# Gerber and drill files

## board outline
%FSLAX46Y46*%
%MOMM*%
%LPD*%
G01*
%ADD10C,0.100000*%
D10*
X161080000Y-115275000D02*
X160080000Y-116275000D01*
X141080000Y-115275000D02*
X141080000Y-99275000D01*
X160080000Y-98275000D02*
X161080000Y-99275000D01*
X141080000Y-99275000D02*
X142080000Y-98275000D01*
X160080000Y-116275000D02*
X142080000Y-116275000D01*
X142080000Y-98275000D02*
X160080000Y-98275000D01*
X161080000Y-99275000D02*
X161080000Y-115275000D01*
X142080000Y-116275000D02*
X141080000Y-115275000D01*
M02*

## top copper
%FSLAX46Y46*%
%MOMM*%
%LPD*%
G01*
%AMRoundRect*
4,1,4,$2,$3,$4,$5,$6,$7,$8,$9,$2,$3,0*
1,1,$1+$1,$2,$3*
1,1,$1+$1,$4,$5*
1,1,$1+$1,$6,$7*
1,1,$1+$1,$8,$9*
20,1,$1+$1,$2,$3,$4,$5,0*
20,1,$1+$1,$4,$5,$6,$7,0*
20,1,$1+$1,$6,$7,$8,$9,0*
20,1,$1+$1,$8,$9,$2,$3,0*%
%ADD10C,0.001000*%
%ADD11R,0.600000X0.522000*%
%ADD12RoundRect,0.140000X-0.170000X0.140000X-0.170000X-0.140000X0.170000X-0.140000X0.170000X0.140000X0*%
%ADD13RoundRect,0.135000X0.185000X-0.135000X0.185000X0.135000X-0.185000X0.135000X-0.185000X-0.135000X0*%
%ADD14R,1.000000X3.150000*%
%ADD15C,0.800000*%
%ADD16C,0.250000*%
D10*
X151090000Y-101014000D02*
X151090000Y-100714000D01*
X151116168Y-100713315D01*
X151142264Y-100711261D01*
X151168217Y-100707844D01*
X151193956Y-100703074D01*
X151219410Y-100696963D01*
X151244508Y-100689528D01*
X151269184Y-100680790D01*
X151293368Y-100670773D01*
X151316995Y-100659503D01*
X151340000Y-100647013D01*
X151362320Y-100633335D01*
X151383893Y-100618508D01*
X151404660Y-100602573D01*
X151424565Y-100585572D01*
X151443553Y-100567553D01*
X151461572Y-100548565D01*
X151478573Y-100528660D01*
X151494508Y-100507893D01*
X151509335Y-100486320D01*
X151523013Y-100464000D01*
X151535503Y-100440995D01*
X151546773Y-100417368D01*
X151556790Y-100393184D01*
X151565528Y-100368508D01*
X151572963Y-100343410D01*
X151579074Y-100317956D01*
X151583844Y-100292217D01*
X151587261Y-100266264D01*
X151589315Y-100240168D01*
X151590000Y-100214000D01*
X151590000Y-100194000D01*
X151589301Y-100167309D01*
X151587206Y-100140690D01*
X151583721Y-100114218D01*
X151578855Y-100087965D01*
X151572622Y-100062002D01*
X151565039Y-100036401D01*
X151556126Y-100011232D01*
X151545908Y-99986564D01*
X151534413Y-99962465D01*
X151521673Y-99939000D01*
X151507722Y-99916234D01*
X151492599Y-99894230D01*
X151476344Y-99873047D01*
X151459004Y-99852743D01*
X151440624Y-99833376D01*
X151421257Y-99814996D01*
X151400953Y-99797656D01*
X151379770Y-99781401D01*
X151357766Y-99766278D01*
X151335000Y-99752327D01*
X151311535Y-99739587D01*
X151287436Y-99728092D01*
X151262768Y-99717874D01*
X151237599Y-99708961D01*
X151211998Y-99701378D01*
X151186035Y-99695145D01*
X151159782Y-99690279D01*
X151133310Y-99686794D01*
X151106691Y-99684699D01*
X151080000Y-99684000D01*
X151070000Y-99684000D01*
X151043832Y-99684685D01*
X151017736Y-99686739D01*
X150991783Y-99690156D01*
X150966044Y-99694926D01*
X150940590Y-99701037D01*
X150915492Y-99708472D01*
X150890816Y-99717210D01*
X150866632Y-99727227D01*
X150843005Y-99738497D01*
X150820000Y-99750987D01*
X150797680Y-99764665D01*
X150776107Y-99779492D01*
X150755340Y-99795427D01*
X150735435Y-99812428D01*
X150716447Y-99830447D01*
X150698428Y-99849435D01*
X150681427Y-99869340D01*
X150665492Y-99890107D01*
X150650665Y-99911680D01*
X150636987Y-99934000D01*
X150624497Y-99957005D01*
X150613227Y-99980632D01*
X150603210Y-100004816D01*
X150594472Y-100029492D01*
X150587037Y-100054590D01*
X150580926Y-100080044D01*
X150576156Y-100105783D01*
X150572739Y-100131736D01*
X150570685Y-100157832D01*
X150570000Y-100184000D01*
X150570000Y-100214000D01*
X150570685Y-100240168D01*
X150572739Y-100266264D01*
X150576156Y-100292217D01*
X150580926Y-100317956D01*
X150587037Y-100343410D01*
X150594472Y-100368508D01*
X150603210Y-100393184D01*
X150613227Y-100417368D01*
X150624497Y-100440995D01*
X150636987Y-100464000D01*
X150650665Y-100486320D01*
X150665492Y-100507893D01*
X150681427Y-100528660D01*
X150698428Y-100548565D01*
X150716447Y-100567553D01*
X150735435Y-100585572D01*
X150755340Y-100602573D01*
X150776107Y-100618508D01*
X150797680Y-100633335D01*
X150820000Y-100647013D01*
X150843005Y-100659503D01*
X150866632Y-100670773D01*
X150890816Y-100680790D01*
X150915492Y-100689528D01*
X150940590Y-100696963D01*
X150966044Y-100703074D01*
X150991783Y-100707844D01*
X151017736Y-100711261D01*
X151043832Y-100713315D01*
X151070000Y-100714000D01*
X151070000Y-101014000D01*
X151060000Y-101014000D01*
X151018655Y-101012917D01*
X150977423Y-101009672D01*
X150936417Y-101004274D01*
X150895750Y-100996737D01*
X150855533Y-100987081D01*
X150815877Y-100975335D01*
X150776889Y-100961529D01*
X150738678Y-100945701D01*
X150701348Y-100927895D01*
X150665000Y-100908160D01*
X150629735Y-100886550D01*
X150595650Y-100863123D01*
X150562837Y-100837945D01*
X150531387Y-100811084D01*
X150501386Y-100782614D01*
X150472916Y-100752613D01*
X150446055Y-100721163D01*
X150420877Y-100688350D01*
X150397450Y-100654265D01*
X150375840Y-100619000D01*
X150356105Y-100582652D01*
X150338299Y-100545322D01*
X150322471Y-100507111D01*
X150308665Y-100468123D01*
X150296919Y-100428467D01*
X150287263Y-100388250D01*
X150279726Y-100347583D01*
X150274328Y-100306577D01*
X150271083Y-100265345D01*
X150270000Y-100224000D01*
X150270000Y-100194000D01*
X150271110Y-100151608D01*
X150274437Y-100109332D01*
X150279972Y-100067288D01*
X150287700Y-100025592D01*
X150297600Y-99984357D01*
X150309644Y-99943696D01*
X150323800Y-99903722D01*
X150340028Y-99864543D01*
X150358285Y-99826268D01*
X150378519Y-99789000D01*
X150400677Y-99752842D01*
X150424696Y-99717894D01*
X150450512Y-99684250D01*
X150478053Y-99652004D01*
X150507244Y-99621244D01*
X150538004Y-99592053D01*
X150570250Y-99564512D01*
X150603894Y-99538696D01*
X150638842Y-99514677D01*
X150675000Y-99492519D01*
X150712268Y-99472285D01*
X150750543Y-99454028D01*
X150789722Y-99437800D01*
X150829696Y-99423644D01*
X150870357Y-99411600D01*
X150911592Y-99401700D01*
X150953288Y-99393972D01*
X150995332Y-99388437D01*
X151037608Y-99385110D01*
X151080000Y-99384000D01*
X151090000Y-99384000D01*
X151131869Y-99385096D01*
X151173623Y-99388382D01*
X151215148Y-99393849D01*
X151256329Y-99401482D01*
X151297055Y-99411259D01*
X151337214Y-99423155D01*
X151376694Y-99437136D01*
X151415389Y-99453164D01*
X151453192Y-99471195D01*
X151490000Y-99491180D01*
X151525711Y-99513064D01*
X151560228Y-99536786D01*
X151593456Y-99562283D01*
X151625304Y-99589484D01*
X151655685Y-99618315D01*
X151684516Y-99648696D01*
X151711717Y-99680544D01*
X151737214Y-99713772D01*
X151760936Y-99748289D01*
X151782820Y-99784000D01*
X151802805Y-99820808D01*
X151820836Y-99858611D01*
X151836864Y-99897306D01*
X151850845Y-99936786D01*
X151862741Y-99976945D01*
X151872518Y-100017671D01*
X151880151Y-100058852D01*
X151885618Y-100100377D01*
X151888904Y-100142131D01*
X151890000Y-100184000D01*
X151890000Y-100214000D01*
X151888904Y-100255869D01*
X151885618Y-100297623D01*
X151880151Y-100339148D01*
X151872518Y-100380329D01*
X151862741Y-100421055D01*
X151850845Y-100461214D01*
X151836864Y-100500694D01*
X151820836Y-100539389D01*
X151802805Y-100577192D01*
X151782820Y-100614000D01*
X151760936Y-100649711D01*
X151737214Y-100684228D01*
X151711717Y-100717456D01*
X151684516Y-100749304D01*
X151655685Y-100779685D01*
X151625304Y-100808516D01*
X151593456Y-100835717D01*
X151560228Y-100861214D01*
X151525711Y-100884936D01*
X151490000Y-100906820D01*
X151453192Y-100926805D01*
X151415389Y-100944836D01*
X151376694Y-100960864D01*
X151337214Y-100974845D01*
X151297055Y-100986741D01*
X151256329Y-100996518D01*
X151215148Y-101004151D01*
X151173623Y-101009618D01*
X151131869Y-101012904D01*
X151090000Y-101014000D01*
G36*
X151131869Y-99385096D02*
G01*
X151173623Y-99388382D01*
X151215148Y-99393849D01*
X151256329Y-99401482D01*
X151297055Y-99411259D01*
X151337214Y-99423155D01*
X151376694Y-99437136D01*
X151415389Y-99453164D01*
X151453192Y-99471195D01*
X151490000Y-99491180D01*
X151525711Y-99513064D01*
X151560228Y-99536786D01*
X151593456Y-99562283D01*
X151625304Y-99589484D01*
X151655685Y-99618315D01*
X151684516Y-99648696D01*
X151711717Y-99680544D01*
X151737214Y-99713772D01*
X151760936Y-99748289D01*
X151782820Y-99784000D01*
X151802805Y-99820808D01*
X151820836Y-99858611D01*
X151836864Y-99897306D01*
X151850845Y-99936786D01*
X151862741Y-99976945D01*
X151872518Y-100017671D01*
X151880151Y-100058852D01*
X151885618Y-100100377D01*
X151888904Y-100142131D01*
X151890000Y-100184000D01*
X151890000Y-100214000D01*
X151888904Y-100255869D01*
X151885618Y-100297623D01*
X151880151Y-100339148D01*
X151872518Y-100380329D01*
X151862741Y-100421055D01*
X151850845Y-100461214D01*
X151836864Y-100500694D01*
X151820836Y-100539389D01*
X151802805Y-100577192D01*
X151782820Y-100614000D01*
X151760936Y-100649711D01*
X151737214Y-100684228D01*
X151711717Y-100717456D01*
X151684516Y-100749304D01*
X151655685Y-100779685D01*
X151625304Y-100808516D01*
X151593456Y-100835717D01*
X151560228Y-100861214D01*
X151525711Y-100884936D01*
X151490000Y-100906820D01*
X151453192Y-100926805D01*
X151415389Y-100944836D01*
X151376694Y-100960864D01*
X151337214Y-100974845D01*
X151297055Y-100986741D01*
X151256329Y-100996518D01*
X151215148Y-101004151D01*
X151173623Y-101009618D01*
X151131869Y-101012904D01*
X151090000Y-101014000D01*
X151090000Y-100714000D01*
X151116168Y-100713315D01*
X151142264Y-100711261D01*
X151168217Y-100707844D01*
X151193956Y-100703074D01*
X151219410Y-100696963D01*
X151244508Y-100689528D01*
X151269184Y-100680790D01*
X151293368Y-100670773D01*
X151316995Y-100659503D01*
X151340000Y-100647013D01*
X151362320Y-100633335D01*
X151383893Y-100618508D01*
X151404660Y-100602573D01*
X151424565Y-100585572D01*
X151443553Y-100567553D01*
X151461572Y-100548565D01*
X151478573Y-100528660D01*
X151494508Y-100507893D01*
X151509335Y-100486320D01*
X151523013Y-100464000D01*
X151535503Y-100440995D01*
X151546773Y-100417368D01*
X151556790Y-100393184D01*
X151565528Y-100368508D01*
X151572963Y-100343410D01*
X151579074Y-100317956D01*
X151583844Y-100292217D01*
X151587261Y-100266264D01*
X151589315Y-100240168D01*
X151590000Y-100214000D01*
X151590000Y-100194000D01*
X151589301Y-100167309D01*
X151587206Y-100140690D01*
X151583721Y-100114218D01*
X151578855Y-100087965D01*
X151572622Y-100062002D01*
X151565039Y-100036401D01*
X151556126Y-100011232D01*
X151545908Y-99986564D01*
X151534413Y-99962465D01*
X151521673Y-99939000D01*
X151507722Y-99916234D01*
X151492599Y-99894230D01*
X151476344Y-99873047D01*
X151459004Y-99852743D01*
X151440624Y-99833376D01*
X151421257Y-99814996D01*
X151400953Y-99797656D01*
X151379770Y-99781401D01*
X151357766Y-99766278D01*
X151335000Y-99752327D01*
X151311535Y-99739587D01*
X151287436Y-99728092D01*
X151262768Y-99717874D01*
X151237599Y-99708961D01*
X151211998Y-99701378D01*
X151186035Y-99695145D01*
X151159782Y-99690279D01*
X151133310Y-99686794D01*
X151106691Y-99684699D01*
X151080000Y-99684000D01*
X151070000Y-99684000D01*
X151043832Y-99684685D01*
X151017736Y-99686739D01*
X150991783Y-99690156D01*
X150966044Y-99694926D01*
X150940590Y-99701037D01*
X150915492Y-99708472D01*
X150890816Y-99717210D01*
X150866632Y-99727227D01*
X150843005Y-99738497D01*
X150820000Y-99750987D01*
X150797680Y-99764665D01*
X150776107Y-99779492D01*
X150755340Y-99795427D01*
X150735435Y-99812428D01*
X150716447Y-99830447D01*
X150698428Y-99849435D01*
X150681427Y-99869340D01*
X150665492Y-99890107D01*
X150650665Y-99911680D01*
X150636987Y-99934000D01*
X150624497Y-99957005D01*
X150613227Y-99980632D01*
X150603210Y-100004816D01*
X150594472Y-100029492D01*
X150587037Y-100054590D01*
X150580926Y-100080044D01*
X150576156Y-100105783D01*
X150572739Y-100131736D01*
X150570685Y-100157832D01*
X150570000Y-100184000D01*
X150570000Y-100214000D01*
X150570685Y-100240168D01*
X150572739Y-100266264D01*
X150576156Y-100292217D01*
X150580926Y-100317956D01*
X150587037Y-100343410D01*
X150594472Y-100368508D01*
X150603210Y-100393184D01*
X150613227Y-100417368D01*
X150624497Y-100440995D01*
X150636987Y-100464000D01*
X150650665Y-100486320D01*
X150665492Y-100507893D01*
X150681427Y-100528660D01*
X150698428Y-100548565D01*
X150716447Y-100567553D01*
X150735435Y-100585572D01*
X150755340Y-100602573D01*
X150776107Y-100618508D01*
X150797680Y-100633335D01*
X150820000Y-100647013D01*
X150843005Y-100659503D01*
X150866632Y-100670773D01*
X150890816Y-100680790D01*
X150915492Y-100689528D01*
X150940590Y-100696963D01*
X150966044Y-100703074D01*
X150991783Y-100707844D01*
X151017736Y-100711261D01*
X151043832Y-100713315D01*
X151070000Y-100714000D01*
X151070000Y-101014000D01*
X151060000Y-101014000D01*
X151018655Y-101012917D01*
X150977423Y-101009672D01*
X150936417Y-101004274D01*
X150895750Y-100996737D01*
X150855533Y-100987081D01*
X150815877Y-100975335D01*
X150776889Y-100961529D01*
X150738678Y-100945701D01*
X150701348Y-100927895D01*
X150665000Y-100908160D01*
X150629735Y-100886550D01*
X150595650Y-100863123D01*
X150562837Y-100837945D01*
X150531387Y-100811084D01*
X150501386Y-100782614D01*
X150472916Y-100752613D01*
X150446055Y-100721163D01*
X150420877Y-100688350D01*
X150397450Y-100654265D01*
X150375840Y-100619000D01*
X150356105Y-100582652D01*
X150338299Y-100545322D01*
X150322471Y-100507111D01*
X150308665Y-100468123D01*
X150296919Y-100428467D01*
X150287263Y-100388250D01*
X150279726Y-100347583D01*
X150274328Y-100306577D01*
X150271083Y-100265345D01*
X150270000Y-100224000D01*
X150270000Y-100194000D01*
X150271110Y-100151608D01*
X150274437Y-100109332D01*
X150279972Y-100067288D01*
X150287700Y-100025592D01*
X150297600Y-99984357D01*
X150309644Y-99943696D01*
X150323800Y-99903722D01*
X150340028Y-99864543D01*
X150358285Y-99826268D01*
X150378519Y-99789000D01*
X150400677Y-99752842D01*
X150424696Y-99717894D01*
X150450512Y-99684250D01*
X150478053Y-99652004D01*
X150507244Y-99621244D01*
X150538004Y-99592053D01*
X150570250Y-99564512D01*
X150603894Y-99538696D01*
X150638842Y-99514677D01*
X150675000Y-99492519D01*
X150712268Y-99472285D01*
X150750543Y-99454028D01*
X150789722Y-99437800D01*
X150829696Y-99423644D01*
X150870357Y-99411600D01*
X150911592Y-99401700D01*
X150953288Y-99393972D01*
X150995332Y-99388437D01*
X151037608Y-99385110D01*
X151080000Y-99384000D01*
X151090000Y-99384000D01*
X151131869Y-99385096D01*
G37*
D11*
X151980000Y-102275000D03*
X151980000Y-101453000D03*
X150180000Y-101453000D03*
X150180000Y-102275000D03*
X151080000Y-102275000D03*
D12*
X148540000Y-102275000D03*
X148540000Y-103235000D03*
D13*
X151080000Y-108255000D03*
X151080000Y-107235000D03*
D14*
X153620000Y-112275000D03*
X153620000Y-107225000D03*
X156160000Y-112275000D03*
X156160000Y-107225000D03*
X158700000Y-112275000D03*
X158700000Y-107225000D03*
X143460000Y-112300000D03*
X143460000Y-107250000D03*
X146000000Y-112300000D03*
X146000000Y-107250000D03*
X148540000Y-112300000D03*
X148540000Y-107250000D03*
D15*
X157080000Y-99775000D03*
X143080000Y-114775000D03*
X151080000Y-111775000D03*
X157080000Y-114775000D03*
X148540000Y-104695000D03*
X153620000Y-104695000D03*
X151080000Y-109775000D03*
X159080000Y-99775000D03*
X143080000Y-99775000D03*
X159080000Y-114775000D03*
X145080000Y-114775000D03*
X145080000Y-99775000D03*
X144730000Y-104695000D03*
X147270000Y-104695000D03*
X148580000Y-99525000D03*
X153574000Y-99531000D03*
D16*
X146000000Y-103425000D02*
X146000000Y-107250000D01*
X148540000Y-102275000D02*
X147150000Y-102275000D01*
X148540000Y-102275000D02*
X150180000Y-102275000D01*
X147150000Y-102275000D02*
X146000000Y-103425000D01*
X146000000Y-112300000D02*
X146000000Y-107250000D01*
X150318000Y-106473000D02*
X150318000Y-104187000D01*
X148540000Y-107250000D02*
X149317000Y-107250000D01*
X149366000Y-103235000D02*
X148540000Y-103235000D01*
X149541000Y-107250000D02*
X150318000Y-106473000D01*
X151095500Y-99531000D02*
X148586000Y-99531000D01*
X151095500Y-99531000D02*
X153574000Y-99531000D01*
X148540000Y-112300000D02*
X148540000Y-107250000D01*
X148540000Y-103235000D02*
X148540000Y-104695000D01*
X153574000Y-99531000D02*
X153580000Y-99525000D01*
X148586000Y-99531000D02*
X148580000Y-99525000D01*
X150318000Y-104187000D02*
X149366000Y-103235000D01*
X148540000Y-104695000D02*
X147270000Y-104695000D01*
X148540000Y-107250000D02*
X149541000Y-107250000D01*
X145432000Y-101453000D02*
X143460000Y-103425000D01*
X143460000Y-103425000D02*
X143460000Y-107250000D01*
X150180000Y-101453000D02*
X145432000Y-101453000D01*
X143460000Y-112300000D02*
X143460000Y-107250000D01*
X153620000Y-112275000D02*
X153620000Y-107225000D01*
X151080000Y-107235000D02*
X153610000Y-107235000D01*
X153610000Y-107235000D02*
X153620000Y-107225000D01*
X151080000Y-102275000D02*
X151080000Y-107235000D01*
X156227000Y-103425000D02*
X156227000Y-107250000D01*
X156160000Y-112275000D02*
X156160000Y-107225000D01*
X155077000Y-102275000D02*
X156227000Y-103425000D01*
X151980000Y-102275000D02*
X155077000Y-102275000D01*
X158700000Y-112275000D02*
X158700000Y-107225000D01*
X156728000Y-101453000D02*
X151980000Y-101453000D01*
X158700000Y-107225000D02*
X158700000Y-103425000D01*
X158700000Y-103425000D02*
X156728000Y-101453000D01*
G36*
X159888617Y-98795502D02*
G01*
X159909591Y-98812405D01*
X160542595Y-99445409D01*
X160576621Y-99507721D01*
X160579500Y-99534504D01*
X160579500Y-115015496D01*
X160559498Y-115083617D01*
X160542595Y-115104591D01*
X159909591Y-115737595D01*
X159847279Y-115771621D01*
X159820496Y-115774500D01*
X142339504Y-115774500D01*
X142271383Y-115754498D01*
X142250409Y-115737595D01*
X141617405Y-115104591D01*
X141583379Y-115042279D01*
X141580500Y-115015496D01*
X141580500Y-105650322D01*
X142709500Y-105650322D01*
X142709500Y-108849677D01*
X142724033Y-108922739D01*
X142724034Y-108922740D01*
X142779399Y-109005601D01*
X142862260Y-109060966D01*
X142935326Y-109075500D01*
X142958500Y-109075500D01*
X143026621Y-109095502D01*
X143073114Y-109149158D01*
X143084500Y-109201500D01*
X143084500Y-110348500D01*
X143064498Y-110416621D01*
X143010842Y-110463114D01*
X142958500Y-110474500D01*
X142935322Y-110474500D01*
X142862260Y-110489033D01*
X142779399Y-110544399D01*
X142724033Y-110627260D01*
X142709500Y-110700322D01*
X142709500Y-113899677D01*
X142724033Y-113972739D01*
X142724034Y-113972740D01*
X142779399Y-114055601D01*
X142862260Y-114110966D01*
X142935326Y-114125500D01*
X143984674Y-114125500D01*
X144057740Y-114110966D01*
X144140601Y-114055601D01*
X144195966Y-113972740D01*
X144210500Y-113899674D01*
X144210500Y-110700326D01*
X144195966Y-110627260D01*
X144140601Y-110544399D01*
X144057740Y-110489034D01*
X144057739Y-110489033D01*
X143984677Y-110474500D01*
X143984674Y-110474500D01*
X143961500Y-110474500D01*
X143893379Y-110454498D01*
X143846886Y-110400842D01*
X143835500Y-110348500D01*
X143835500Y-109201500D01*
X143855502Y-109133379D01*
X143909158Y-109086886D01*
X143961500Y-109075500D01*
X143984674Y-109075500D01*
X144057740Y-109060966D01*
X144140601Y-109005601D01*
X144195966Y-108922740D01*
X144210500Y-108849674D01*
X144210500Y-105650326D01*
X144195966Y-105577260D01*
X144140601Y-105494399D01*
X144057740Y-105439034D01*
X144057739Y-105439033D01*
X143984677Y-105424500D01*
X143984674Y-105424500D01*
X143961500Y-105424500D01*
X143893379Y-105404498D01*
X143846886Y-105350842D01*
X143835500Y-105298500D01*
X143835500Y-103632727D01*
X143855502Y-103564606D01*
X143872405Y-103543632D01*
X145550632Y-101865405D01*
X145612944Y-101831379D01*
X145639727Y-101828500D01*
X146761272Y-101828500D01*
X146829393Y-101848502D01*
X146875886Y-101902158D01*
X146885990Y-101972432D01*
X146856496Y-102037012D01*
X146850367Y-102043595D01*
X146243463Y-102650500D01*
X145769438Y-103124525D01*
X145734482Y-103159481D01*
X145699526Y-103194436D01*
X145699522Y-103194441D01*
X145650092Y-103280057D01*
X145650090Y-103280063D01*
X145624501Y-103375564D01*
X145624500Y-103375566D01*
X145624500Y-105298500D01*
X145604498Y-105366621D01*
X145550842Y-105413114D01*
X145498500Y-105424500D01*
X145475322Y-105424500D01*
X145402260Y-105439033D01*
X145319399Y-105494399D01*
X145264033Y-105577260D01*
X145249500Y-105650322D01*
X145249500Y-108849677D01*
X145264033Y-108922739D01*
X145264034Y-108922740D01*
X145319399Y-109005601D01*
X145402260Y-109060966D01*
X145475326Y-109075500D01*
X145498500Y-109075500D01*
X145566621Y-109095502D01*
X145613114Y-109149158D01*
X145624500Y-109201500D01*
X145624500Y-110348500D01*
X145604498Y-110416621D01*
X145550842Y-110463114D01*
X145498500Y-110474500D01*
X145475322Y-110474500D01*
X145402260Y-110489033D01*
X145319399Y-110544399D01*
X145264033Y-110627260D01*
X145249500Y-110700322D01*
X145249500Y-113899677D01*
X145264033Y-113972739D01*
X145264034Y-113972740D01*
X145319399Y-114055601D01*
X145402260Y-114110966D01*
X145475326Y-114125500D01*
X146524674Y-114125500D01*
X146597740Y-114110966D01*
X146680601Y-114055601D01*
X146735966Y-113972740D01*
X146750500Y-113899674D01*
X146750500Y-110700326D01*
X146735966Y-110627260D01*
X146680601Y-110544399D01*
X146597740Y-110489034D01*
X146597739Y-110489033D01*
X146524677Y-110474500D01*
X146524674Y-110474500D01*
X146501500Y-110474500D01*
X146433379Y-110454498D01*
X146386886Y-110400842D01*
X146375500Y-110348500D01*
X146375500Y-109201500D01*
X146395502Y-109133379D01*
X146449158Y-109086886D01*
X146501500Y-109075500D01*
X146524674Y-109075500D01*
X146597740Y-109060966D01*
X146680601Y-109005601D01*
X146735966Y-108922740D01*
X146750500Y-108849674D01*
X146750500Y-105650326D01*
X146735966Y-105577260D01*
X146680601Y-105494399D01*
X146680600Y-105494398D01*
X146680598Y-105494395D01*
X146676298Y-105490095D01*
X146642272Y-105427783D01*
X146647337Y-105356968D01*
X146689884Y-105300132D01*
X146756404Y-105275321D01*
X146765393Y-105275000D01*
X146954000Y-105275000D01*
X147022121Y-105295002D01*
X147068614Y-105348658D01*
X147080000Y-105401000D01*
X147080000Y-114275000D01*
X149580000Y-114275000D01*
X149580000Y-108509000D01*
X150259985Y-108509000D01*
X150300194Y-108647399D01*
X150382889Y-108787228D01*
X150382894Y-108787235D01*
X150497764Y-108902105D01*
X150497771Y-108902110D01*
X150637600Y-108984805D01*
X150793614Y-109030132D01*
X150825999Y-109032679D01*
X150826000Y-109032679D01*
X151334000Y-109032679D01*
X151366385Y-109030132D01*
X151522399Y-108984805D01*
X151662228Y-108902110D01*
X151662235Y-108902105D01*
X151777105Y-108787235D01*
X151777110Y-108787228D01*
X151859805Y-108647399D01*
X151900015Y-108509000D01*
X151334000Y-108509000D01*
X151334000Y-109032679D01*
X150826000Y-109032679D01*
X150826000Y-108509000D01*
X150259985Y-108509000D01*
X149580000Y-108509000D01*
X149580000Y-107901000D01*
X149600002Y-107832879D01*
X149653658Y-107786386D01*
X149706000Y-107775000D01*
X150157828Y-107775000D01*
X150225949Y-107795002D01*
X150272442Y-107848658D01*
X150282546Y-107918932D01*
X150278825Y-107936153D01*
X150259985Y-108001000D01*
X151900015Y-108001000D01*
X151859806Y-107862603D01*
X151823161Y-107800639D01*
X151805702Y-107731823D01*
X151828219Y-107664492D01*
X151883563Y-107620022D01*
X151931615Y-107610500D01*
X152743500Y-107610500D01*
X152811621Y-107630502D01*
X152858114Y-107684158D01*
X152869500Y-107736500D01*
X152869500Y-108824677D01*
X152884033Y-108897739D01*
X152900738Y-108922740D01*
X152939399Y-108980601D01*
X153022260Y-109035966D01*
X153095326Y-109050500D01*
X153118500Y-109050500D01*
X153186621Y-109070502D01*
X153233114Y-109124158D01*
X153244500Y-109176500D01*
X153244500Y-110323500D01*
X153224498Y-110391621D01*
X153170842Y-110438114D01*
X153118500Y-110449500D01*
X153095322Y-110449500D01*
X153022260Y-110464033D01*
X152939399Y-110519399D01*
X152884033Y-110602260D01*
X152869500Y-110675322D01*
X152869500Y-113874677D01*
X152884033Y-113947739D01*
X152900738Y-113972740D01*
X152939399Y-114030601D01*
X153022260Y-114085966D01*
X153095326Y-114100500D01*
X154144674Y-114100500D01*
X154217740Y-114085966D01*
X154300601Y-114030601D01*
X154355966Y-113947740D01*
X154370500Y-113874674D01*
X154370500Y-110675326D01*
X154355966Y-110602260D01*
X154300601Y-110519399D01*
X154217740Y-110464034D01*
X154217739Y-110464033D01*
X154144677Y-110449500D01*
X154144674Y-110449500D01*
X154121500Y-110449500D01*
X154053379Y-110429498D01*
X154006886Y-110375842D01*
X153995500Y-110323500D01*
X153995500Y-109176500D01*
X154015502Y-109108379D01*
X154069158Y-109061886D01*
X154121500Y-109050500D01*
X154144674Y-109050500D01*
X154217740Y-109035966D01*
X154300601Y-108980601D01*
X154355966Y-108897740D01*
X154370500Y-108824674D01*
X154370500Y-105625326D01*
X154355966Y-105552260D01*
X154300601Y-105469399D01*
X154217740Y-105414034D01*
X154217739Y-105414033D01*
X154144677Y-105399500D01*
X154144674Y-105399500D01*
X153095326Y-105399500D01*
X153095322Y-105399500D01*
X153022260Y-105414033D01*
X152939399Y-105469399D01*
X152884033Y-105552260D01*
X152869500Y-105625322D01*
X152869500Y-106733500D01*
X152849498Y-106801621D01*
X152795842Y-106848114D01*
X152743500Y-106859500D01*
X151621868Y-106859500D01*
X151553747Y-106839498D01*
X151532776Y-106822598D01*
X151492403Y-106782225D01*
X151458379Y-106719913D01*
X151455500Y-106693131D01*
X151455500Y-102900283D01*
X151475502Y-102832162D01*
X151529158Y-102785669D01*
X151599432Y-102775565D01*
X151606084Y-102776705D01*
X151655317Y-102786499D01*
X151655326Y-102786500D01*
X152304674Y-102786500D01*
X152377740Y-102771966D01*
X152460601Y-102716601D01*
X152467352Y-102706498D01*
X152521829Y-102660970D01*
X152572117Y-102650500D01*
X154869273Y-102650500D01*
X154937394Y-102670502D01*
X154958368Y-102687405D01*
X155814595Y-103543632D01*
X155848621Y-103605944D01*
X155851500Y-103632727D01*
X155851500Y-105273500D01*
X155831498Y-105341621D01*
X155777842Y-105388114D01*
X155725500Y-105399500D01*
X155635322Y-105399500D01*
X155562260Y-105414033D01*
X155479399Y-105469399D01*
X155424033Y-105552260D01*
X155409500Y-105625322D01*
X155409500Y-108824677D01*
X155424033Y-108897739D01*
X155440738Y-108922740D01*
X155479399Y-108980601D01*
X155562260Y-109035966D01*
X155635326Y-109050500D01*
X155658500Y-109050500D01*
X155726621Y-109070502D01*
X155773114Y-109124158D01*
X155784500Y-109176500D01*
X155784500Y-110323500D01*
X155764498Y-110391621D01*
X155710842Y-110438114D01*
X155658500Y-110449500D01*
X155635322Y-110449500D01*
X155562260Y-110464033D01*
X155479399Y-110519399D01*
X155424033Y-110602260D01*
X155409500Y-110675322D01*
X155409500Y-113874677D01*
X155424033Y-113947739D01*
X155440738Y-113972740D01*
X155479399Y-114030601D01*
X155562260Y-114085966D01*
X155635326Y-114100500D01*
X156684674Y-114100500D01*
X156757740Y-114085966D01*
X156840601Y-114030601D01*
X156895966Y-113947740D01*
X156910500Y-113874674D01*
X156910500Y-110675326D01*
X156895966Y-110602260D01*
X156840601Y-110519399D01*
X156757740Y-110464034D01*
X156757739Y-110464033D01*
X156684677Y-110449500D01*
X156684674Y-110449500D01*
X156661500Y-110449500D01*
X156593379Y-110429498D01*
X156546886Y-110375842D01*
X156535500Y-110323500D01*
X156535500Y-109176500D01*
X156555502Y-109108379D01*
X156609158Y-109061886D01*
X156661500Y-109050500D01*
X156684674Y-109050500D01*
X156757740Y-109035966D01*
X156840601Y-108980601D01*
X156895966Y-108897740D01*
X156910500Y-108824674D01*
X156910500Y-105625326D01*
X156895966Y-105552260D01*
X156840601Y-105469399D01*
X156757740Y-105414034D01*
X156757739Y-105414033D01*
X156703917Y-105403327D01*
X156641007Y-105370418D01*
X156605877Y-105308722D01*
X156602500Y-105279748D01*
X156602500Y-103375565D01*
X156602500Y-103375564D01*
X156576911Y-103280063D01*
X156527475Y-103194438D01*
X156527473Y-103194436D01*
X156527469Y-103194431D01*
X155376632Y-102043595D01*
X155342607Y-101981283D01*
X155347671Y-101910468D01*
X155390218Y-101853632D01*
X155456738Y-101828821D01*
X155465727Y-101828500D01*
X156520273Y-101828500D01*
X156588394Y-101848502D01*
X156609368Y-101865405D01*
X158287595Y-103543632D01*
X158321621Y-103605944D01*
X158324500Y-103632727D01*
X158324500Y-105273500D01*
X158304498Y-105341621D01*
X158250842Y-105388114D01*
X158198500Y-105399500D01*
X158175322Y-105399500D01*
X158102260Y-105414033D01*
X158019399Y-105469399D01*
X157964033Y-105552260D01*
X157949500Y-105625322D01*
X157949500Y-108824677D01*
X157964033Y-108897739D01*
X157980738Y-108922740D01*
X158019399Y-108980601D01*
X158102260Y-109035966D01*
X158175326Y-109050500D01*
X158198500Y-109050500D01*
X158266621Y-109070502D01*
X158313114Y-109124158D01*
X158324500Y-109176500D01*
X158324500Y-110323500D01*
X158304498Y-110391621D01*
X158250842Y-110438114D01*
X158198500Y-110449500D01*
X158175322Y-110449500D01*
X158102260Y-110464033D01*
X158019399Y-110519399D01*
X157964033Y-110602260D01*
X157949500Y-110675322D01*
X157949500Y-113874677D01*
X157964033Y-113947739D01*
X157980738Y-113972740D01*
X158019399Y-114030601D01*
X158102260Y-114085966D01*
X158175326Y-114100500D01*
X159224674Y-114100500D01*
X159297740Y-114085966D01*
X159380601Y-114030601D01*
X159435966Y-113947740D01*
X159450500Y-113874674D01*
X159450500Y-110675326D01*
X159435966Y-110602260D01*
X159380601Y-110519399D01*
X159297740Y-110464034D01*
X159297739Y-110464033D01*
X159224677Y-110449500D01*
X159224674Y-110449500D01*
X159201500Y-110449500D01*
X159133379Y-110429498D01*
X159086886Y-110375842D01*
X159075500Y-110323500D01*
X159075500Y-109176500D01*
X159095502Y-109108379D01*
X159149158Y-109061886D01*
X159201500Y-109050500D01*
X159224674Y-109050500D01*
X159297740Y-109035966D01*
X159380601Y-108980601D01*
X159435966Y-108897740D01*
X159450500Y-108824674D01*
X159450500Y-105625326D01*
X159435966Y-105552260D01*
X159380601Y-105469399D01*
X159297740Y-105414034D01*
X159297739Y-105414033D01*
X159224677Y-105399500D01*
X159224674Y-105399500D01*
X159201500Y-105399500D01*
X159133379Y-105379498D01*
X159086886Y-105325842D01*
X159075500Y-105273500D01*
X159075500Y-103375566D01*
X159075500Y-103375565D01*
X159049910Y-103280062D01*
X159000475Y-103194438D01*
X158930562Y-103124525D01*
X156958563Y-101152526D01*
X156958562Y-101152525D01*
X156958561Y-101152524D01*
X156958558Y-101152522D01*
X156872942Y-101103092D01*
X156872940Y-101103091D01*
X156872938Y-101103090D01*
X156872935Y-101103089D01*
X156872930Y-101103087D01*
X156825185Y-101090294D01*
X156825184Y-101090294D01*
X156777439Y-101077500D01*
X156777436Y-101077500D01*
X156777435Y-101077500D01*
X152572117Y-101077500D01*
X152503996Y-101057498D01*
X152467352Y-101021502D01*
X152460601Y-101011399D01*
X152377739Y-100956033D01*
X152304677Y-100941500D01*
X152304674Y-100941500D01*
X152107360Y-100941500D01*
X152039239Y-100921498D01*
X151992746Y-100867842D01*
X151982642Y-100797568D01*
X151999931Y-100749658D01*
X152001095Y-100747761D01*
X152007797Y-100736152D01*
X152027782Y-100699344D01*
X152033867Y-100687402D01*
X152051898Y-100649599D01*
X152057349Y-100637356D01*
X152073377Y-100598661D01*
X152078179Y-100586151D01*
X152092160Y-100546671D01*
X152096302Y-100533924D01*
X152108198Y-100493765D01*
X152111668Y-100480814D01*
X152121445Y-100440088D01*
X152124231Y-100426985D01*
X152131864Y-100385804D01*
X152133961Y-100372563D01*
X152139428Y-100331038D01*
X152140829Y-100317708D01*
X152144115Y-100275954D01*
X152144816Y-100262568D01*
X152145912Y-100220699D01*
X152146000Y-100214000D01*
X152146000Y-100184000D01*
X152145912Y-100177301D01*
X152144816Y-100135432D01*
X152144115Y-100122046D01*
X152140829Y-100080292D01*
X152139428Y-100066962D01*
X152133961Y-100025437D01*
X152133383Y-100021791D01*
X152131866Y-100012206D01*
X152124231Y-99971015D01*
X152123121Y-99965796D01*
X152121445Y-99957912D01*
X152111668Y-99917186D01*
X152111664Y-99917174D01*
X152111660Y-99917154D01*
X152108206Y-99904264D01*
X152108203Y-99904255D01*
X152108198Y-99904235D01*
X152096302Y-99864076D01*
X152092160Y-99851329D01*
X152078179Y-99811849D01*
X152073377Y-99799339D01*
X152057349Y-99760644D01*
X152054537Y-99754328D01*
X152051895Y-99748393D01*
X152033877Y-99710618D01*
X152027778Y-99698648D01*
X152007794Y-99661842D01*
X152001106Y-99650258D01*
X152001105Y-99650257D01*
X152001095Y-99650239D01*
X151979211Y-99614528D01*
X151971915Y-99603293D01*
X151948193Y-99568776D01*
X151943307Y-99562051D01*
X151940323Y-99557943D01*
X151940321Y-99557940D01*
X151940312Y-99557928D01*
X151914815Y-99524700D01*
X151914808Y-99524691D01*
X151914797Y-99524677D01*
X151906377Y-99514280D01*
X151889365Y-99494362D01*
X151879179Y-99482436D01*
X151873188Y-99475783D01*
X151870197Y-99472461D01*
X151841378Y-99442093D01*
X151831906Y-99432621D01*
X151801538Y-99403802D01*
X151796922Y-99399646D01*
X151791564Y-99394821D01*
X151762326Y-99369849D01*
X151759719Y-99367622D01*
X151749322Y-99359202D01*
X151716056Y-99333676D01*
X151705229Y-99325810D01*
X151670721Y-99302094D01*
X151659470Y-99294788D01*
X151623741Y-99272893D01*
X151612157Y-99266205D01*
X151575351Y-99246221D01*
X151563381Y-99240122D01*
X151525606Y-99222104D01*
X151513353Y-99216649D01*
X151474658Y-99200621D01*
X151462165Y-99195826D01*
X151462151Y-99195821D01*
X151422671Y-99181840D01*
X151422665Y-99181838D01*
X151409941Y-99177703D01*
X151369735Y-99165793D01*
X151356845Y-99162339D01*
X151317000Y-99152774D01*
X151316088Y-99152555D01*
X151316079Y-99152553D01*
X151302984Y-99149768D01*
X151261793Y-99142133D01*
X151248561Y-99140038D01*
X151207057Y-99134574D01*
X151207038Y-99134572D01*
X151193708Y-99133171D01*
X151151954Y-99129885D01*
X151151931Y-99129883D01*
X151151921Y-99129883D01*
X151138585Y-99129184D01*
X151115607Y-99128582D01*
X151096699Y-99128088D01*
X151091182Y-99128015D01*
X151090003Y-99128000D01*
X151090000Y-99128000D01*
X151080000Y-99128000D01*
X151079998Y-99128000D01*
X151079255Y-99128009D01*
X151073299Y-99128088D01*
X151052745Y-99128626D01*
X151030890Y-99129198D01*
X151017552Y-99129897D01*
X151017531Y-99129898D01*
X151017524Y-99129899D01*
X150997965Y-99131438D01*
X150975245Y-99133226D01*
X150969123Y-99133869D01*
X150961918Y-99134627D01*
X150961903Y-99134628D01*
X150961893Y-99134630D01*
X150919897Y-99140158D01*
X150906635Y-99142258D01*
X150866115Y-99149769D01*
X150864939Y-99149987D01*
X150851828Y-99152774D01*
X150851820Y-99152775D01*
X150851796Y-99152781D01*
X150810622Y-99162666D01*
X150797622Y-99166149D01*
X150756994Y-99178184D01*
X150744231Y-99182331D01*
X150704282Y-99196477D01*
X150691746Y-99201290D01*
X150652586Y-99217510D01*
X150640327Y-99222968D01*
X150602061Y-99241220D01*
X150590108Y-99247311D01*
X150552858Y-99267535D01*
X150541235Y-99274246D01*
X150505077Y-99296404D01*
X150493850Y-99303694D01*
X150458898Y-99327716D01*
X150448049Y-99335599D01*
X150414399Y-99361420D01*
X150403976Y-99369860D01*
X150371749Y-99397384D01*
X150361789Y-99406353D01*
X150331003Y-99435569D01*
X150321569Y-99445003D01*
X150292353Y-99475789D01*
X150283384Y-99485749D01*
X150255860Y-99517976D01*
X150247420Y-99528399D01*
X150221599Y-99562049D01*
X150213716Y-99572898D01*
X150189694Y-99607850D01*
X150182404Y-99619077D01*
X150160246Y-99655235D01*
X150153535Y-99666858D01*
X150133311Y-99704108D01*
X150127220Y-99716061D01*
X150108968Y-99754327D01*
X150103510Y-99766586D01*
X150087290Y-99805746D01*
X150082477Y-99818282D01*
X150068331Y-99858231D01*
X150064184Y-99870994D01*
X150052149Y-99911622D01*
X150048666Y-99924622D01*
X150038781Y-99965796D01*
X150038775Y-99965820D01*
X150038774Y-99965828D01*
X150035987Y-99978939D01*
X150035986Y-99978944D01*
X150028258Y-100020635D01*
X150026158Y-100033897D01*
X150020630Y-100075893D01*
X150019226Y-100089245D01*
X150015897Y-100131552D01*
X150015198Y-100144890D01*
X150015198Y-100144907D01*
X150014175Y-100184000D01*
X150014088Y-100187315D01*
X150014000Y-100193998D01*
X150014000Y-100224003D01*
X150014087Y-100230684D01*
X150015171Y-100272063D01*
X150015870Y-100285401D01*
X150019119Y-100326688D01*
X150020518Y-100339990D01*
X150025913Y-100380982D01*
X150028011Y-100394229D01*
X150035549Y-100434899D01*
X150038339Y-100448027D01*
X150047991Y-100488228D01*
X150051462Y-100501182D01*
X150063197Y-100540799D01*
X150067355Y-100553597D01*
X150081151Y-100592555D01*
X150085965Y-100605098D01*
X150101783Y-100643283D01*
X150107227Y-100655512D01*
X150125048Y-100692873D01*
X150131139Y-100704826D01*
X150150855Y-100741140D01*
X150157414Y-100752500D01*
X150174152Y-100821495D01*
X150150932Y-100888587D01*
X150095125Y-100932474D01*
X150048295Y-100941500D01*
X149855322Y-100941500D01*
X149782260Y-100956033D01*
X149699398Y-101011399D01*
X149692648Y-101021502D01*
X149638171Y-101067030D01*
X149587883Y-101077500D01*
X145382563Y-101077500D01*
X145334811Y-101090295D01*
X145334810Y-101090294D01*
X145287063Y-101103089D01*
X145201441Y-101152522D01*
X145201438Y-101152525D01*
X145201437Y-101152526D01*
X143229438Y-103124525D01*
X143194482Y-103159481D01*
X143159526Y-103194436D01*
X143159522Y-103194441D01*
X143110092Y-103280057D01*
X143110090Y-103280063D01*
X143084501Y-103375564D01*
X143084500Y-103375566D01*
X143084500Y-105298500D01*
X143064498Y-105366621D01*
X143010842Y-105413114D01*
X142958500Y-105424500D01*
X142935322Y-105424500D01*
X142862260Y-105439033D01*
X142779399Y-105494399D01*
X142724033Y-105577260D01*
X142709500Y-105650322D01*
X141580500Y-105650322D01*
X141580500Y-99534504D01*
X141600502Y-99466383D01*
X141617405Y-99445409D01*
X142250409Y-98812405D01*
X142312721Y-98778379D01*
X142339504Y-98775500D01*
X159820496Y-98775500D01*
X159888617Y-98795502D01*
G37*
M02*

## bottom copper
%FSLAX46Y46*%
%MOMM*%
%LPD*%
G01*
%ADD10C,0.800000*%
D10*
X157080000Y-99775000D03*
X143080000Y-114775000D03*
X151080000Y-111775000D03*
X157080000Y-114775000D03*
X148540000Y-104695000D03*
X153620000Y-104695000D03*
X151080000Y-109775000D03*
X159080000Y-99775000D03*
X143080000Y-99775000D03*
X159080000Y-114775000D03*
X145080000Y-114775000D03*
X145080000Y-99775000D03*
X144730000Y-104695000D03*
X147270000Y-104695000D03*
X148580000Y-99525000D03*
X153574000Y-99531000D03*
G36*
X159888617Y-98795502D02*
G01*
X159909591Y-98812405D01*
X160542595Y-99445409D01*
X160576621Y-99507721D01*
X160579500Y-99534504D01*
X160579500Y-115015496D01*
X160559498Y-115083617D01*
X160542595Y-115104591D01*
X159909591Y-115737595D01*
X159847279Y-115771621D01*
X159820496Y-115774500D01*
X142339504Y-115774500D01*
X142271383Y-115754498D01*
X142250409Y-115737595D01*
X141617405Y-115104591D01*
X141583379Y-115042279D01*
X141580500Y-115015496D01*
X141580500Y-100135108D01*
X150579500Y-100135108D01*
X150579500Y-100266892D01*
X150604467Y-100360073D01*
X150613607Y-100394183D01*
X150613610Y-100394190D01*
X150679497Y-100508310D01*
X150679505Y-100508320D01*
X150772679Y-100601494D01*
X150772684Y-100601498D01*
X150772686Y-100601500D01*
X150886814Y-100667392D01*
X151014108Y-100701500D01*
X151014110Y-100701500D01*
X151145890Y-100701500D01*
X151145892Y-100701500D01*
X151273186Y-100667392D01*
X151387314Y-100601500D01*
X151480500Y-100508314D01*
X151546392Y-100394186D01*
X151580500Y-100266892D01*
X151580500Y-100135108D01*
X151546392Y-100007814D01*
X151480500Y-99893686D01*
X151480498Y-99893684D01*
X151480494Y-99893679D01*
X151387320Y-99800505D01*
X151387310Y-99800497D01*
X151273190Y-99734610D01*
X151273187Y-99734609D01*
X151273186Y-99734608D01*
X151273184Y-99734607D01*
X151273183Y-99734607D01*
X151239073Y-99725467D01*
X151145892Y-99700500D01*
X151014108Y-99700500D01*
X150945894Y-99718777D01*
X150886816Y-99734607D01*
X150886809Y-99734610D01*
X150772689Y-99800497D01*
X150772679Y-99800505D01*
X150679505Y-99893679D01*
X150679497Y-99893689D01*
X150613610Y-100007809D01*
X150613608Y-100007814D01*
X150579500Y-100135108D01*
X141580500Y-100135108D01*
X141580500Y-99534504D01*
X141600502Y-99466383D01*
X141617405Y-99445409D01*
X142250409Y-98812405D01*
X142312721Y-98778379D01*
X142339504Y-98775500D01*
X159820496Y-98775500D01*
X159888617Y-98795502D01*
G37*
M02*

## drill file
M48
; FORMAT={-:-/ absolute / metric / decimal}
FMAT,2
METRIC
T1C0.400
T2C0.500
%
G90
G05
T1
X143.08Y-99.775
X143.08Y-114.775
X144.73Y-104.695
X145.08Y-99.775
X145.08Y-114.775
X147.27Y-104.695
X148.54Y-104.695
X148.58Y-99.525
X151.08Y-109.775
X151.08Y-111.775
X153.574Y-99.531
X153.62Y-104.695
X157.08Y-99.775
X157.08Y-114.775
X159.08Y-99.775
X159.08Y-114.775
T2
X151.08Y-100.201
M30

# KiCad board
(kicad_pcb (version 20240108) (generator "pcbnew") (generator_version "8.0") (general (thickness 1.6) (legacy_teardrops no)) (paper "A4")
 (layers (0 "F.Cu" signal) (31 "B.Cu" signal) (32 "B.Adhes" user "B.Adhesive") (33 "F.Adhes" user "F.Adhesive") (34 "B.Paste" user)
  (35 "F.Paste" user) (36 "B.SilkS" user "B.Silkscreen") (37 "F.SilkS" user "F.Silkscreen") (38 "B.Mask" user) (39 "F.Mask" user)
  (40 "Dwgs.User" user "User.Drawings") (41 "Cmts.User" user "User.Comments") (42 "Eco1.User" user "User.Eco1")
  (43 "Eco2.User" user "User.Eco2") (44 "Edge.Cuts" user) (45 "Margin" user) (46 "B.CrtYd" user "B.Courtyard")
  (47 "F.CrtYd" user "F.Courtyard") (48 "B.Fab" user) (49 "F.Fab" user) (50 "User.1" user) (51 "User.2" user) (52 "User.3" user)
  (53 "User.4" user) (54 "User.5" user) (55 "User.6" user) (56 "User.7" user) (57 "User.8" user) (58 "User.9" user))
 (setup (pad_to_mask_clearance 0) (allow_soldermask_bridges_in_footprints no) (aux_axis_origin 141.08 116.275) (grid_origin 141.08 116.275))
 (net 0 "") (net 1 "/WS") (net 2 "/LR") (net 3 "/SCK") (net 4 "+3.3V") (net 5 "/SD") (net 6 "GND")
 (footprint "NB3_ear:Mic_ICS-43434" (layer "F.Cu") (at 151.08 100.914 180)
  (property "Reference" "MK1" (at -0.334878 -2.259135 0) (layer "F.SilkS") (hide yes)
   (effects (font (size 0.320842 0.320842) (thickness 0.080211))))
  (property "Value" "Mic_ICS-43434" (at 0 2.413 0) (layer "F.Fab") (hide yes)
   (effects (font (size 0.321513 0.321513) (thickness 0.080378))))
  (fp_poly
   (pts (xy -0.01 -0.1) (xy -0.01 0.2) (xy -0.036168 0.200685) (xy -0.062264 0.202739) (xy -0.088217 0.206156) (xy -0.113956 0.210926)
    (xy -0.13941 0.217037) (xy -0.164508 0.224472) (xy -0.189184 0.23321) (xy -0.213368 0.243227) (xy -0.236995 0.254497)
    (xy -0.26 0.266987) (xy -0.28232 0.280665) (xy -0.303893 0.295492) (xy -0.32466 0.311427) (xy -0.344565 0.328428)
    (xy -0.363553 0.346447) (xy -0.381572 0.365435) (xy -0.398573 0.38534) (xy -0.414508 0.406107) (xy -0.429335 0.42768)
    (xy -0.443013 0.45) (xy -0.455503 0.473005) (xy -0.466773 0.496632) (xy -0.47679 0.520816) (xy -0.485528 0.545492)
    (xy -0.492963 0.57059) (xy -0.499074 0.596044) (xy -0.503844 0.621783) (xy -0.507261 0.647736) (xy -0.509315 0.673832) (xy -0.51 0.7)
    (xy -0.51 0.72) (xy -0.509301 0.746691) (xy -0.507206 0.77331) (xy -0.503721 0.799782) (xy -0.498855 0.826035) (xy -0.492622 0.851998)
    (xy -0.485039 0.877599) (xy -0.476126 0.902768) (xy -0.465908 0.927436) (xy -0.454413 0.951535) (xy -0.441673 0.975)
    (xy -0.427722 0.997766) (xy -0.412599 1.01977) (xy -0.396344 1.040953) (xy -0.379004 1.061257) (xy -0.360624 1.080624)
    (xy -0.341257 1.099004) (xy -0.320953 1.116344) (xy -0.29977 1.132599) (xy -0.277766 1.147722) (xy -0.255 1.161673)
    (xy -0.231535 1.174413) (xy -0.207436 1.185908) (xy -0.182768 1.196126) (xy -0.157599 1.205039) (xy -0.131998 1.212622)
    (xy -0.106035 1.218855) (xy -0.079782 1.223721) (xy -0.05331 1.227206) (xy -0.026691 1.229301) (xy 0 1.23) (xy 0.01 1.23)
    (xy 0.036168 1.229315) (xy 0.062264 1.227261) (xy 0.088217 1.223844) (xy 0.113956 1.219074) (xy 0.13941 1.212963) (xy 0.164508 1.205528)
    (xy 0.189184 1.19679) (xy 0.213368 1.186773) (xy 0.236995 1.175503) (xy 0.26 1.163013) (xy 0.28232 1.149335) (xy 0.303893 1.134508)
    (xy 0.32466 1.118573) (xy 0.344565 1.101572) (xy 0.363553 1.083553) (xy 0.381572 1.064565) (xy 0.398573 1.04466) (xy 0.414508 1.023893)
    (xy 0.429335 1.00232) (xy 0.443013 0.98) (xy 0.455503 0.956995) (xy 0.466773 0.933368) (xy 0.47679 0.909184) (xy 0.485528 0.884508)
    (xy 0.492963 0.85941) (xy 0.499074 0.833956) (xy 0.503844 0.808217) (xy 0.507261 0.782264) (xy 0.509315 0.756168) (xy 0.51 0.73)
    (xy 0.51 0.7) (xy 0.509315 0.673832) (xy 0.507261 0.647736) (xy 0.503844 0.621783) (xy 0.499074 0.596044) (xy 0.492963 0.57059)
    (xy 0.485528 0.545492) (xy 0.47679 0.520816) (xy 0.466773 0.496632) (xy 0.455503 0.473005) (xy 0.443013 0.45) (xy 0.429335 0.42768)
    (xy 0.414508 0.406107) (xy 0.398573 0.38534) (xy 0.381572 0.365435) (xy 0.363553 0.346447) (xy 0.344565 0.328428) (xy 0.32466 0.311427)
    (xy 0.303893 0.295492) (xy 0.28232 0.280665) (xy 0.26 0.266987) (xy 0.236995 0.254497) (xy 0.213368 0.243227) (xy 0.189184 0.23321)
    (xy 0.164508 0.224472) (xy 0.13941 0.217037) (xy 0.113956 0.210926) (xy 0.088217 0.206156) (xy 0.062264 0.202739) (xy 0.036168 0.200685)
    (xy 0.01 0.2) (xy 0.01 -0.1) (xy 0.02 -0.1) (xy 0.061345 -0.098917) (xy 0.102577 -0.095672) (xy 0.143583 -0.090274)
    (xy 0.18425 -0.082737) (xy 0.224467 -0.073081) (xy 0.264123 -0.061335) (xy 0.303111 -0.047529) (xy 0.341322 -0.031701)
    (xy 0.378652 -0.013895) (xy 0.415 0.00584) (xy 0.450265 0.02745) (xy 0.48435 0.050877) (xy 0.517163 0.076055) (xy 0.548613 0.102916)
    (xy 0.578614 0.131386) (xy 0.607084 0.161387) (xy 0.633945 0.192837) (xy 0.659123 0.22565) (xy 0.68255 0.259735) (xy 0.70416 0.295)
    (xy 0.723895 0.331348) (xy 0.741701 0.368678) (xy 0.757529 0.406889) (xy 0.771335 0.445877) (xy 0.783081 0.485533) (xy 0.792737 0.52575)
    (xy 0.800274 0.566417) (xy 0.805672 0.607423) (xy 0.808917 0.648655) (xy 0.81 0.69) (xy 0.81 0.72) (xy 0.80889 0.762392)
    (xy 0.805563 0.804668) (xy 0.800028 0.846712) (xy 0.7923 0.888408) (xy 0.7824 0.929643) (xy 0.770356 0.970304) (xy 0.7562 1.010278)
    (xy 0.739972 1.049457) (xy 0.721715 1.087732) (xy 0.701481 1.125) (xy 0.679323 1.161158) (xy 0.655304 1.196106) (xy 0.629488 1.22975)
    (xy 0.601947 1.261996) (xy 0.572756 1.292756) (xy 0.541996 1.321947) (xy 0.50975 1.349488) (xy 0.476106 1.375304) (xy 0.441158 1.399323)
    (xy 0.405 1.421481) (xy 0.367732 1.441715) (xy 0.329457 1.459972) (xy 0.290278 1.4762) (xy 0.250304 1.490356) (xy 0.209643 1.5024)
    (xy 0.168408 1.5123) (xy 0.126712 1.520028) (xy 0.084668 1.525563) (xy 0.042392 1.52889) (xy 0 1.53) (xy -0.01 1.53)
    (xy -0.051869 1.528904) (xy -0.093623 1.525618) (xy -0.135148 1.520151) (xy -0.176329 1.512518) (xy -0.217055 1.502741)
    (xy -0.257214 1.490845) (xy -0.296694 1.476864) (xy -0.335389 1.460836) (xy -0.373192 1.442805) (xy -0.41 1.42282)
    (xy -0.445711 1.400936) (xy -0.480228 1.377214) (xy -0.513456 1.351717) (xy -0.545304 1.324516) (xy -0.575685 1.295685)
    (xy -0.604516 1.265304) (xy -0.631717 1.233456) (xy -0.657214 1.200228) (xy -0.680936 1.165711) (xy -0.70282 1.13)
    (xy -0.722805 1.093192) (xy -0.740836 1.055389) (xy -0.756864 1.016694) (xy -0.770845 0.977214) (xy -0.782741 0.937055)
    (xy -0.792518 0.896329) (xy -0.800151 0.855148) (xy -0.805618 0.813623) (xy -0.808904 0.771869) (xy -0.81 0.73) (xy -0.81 0.7)
    (xy -0.808904 0.658131) (xy -0.805618 0.616377) (xy -0.800151 0.574852) (xy -0.792518 0.533671) (xy -0.782741 0.492945)
    (xy -0.770845 0.452786) (xy -0.756864 0.413306) (xy -0.740836 0.374611) (xy -0.722805 0.336808) (xy -0.70282 0.3)
    (xy -0.680936 0.264289) (xy -0.657214 0.229772) (xy -0.631717 0.196544) (xy -0.604516 0.164696) (xy -0.575685 0.134315)
    (xy -0.545304 0.105484) (xy -0.513456 0.078283) (xy -0.480228 0.052786) (xy -0.445711 0.029064) (xy -0.41 0.00718)
    (xy -0.373192 -0.012805) (xy -0.335389 -0.030836) (xy -0.296694 -0.046864) (xy -0.257214 -0.060845) (xy -0.217055 -0.072741)
    (xy -0.176329 -0.082518) (xy -0.135148 -0.090151) (xy -0.093623 -0.095618) (xy -0.051869 -0.098904) (xy -0.01 -0.1))
   (stroke (width 0.001) (type solid)) (fill solid) (layer "F.Cu"))
  (pad "" np_thru_hole circle (at 0 0.713 180) (size 0.5 0.5) (drill 0.5) (layers "*.Cu" "*.Mask"))
  (pad "1" smd rect (at -0.9 -1.361 180) (size 0.6 0.522) (layers "F.Cu" "F.Mask") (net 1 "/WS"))
  (pad "2" smd rect (at -0.9 -0.539 180) (size 0.6 0.522) (layers "F.Cu" "F.Mask") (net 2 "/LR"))
  (pad "4" smd rect (at 0.9 -0.539 180) (size 0.6 0.522) (layers "F.Cu" "F.Mask") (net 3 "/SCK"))
  (pad "5" smd rect (at 0.9 -1.361 180) (size 0.6 0.522) (layers "F.Cu" "F.Mask") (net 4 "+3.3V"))
  (pad "6" smd rect (at 0 -1.361 180) (size 0.6 0.522) (layers "F.Cu" "F.Mask") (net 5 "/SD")))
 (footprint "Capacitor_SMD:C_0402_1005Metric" (layer "F.Cu") (at 148.54 102.755 -90)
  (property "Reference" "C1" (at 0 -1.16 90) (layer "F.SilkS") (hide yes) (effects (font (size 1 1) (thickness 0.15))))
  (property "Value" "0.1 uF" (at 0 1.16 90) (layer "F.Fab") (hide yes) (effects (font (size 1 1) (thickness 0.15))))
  (pad "1" smd roundrect (at -0.48 0 270) (size 0.56 0.62) (layers "F.Cu" "F.Paste" "F.Mask") (roundrect_rratio 0.25) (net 4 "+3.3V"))
  (pad "2" smd roundrect (at 0.48 0 270) (size 0.56 0.62) (layers "F.Cu" "F.Paste" "F.Mask") (roundrect_rratio 0.25) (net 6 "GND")))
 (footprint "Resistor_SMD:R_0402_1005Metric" (layer "F.Cu") (at 151.08 107.745 90)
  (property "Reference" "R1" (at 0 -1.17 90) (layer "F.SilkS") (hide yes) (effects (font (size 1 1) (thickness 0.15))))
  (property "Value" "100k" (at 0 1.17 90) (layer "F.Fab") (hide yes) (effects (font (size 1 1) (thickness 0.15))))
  (pad "1" smd roundrect (at -0.51 0 90) (size 0.54 0.64) (layers "F.Cu" "F.Paste" "F.Mask") (roundrect_rratio 0.25) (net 6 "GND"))
  (pad "2" smd roundrect (at 0.51 0 90) (size 0.54 0.64) (layers "F.Cu" "F.Paste" "F.Mask") (roundrect_rratio 0.25) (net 5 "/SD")))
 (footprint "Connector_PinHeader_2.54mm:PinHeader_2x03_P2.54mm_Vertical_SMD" (layer "F.Cu") (at 156.16 109.75 90)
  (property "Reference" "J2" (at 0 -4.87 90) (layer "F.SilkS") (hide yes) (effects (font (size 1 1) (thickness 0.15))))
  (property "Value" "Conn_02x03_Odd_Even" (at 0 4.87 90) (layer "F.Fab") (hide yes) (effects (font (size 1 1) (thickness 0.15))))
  (pad "1" smd rect (at -2.525 -2.54 90) (size 3.15 1) (layers "F.Cu" "F.Paste" "F.Mask") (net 5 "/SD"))
  (pad "2" smd rect (at 2.525 -2.54 90) (size 3.15 1) (layers "F.Cu" "F.Paste" "F.Mask") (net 5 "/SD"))
  (pad "3" smd rect (at -2.525 0 90) (size 3.15 1) (layers "F.Cu" "F.Paste" "F.Mask") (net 1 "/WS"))
  (pad "4" smd rect (at 2.525 0 90) (size 3.15 1) (layers "F.Cu" "F.Paste" "F.Mask") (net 1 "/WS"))
  (pad "5" smd rect (at -2.525 2.54 90) (size 3.15 1) (layers "F.Cu" "F.Paste" "F.Mask") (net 2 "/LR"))
  (pad "6" smd rect (at 2.525 2.54 90) (size 3.15 1) (layers "F.Cu" "F.Paste" "F.Mask") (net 2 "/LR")))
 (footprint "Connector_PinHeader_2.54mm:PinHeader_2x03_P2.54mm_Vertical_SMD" (layer "F.Cu") (at 146 109.775 90)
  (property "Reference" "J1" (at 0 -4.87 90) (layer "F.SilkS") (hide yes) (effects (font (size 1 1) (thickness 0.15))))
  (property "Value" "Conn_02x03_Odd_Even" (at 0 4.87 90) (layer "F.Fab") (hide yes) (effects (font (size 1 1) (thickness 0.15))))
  (pad "1" smd rect (at -2.525 -2.54 90) (size 3.15 1) (layers "F.Cu" "F.Paste" "F.Mask") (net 3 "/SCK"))
  (pad "2" smd rect (at 2.525 -2.54 90) (size 3.15 1) (layers "F.Cu" "F.Paste" "F.Mask") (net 3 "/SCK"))
  (pad "3" smd rect (at -2.525 0 90) (size 3.15 1) (layers "F.Cu" "F.Paste" "F.Mask") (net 4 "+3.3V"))
  (pad "4" smd rect (at 2.525 0 90) (size 3.15 1) (layers "F.Cu" "F.Paste" "F.Mask") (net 4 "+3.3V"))
  (pad "5" smd rect (at -2.525 2.54 90) (size 3.15 1) (layers "F.Cu" "F.Paste" "F.Mask") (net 6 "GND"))
  (pad "6" smd rect (at 2.525 2.54 90) (size 3.15 1) (layers "F.Cu" "F.Paste" "F.Mask") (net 6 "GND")))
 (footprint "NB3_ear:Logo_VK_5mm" (layer "B.Cu") (at 151.08 107.275 180)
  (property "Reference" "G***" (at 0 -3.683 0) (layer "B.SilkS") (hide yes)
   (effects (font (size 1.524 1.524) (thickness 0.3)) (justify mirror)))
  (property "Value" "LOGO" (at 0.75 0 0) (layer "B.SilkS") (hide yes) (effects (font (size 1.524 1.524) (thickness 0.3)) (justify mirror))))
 (gr_line (start 161.08 115.275) (end 160.08 116.275) (stroke (width 0.1) (type default)) (layer "Edge.Cuts"))
 (gr_line (start 141.08 115.275) (end 141.08 99.275) (stroke (width 0.1) (type default)) (layer "Edge.Cuts"))
 (gr_line (start 160.08 98.275) (end 161.08 99.275) (stroke (width 0.1) (type default)) (layer "Edge.Cuts"))
 (gr_line (start 141.08 99.275) (end 142.08 98.275) (stroke (width 0.1) (type default)) (layer "Edge.Cuts"))
 (gr_line (start 160.08 116.275) (end 142.08 116.275) (stroke (width 0.1) (type default)) (layer "Edge.Cuts"))
 (gr_line (start 142.08 98.275) (end 160.08 98.275) (stroke (width 0.1) (type default)) (layer "Edge.Cuts"))
 (gr_line (start 161.08 99.275) (end 161.08 115.275) (stroke (width 0.1) (type default)) (layer "Edge.Cuts"))
 (gr_line (start 142.08 116.275) (end 141.08 115.275) (stroke (width 0.1) (type default)) (layer "Edge.Cuts"))
 (segment (start 146 103.425) (end 146 107.25) (width 0.25) (layer "F.Cu") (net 4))
 (segment (start 148.54 102.275) (end 147.15 102.275) (width 0.25) (layer "F.Cu") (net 4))
 (segment (start 148.54 102.275) (end 150.18 102.275) (width 0.25) (layer "F.Cu") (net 4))
 (segment (start 147.15 102.275) (end 146 103.425) (width 0.25) (layer "F.Cu") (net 4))
 (segment (start 146 112.3) (end 146 107.25) (width 0.25) (layer "F.Cu") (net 4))
 (segment (start 150.318 106.473) (end 150.318 104.187) (width 0.25) (layer "F.Cu") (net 6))
 (segment (start 148.54 107.25) (end 149.317 107.25) (width 0.25) (layer "F.Cu") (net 6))
 (segment (start 149.366 103.235) (end 148.54 103.235) (width 0.25) (layer "F.Cu") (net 6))
 (segment (start 149.541 107.25) (end 150.318 106.473) (width 0.25) (layer "F.Cu") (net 6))
 (segment (start 151.0955 99.531) (end 148.586 99.531) (width 0.25) (layer "F.Cu") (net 6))
 (segment (start 151.0955 99.531) (end 153.574 99.531) (width 0.25) (layer "F.Cu") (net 6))
 (segment (start 148.54 112.3) (end 148.54 107.25) (width 0.25) (layer "F.Cu") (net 6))
 (segment (start 148.54 103.235) (end 148.54 104.695) (width 0.25) (layer "F.Cu") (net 6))
 (segment (start 153.574 99.531) (end 153.58 99.525) (width 0.25) (layer "F.Cu") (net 6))
 (segment (start 148.586 99.531) (end 148.58 99.525) (width 0.25) (layer "F.Cu") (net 6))
 (segment (start 150.318 104.187) (end 149.366 103.235) (width 0.25) (layer "F.Cu") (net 6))
 (segment (start 148.54 104.695) (end 147.27 104.695) (width 0.25) (layer "F.Cu") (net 6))
 (segment (start 148.54 107.25) (end 149.541 107.25) (width 0.25) (layer "F.Cu") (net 6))
 (via (at 157.08 99.775) (size 0.8) (drill 0.4) (layers "F.Cu" "B.Cu") (free yes) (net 6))
 (via (at 143.08 114.775) (size 0.8) (drill 0.4) (layers "F.Cu" "B.Cu") (free yes) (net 6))
 (via (at 151.08 111.775) (size 0.8) (drill 0.4) (layers "F.Cu" "B.Cu") (free yes) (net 6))
 (via (at 157.08 114.775) (size 0.8) (drill 0.4) (layers "F.Cu" "B.Cu") (free yes) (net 6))
 (via (at 148.54 104.695) (size 0.8) (drill 0.4) (layers "F.Cu" "B.Cu") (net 6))
 (via (at 153.62 104.695) (size 0.8) (drill 0.4) (layers "F.Cu" "B.Cu") (free yes) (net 6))
 (via (at 151.08 109.775) (size 0.8) (drill 0.4) (layers "F.Cu" "B.Cu") (free yes) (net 6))
 (via (at 159.08 99.775) (size 0.8) (drill 0.4) (layers "F.Cu" "B.Cu") (free yes) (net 6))
 (via (at 143.08 99.775) (size 0.8) (drill 0.4) (layers "F.Cu" "B.Cu") (free yes) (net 6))
 (via (at 159.08 114.775) (size 0.8) (drill 0.4) (layers "F.Cu" "B.Cu") (free yes) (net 6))
 (via (at 145.08 114.775) (size 0.8) (drill 0.4) (layers "F.Cu" "B.Cu") (free yes) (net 6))
 (via (at 145.08 99.775) (size 0.8) (drill 0.4) (layers "F.Cu" "B.Cu") (free yes) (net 6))
 (via (at 144.73 104.695) (size 0.8) (drill 0.4) (layers "F.Cu" "B.Cu") (free yes) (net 6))
 (via (at 147.27 104.695) (size 0.8) (drill 0.4) (layers "F.Cu" "B.Cu") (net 6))
 (via (at 148.58 99.525) (size 0.8) (drill 0.4) (layers "F.Cu" "B.Cu") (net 6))
 (via (at 153.574 99.531) (size 0.8) (drill 0.4) (layers "F.Cu" "B.Cu") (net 6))
 (segment (start 145.432 101.453) (end 143.46 103.425) (width 0.25) (layer "F.Cu") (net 3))
 (segment (start 143.46 103.425) (end 143.46 107.25) (width 0.25) (layer "F.Cu") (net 3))
 (segment (start 150.18 101.453) (end 145.432 101.453) (width 0.25) (layer "F.Cu") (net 3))
 (segment (start 143.46 112.3) (end 143.46 107.25) (width 0.25) (layer "F.Cu") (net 3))
 (segment (start 153.62 112.275) (end 153.62 107.225) (width 0.25) (layer "F.Cu") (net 5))
 (segment (start 151.08 107.235) (end 153.61 107.235) (width 0.25) (layer "F.Cu") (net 5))
 (segment (start 153.61 107.235) (end 153.62 107.225) (width 0.25) (layer "F.Cu") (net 5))
 (segment (start 151.08 102.275) (end 151.08 107.235) (width 0.25) (layer "F.Cu") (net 5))
 (segment (start 156.227 103.425) (end 156.227 107.25) (width 0.25) (layer "F.Cu") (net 1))
 (segment (start 156.16 112.275) (end 156.16 107.225) (width 0.25) (layer "F.Cu") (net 1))
 (segment (start 155.077 102.275) (end 156.227 103.425) (width 0.25) (layer "F.Cu") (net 1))
 (segment (start 151.98 102.275) (end 155.077 102.275) (width 0.25) (layer "F.Cu") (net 1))
 (segment (start 158.7 112.275) (end 158.7 107.225) (width 0.25) (layer "F.Cu") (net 2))
 (segment (start 156.728 101.453) (end 151.98 101.453) (width 0.25) (layer "F.Cu") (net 2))
 (segment (start 158.7 107.225) (end 158.7 103.425) (width 0.25) (layer "F.Cu") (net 2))
 (segment (start 158.7 103.425) (end 156.728 101.453) (width 0.25) (layer "F.Cu") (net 2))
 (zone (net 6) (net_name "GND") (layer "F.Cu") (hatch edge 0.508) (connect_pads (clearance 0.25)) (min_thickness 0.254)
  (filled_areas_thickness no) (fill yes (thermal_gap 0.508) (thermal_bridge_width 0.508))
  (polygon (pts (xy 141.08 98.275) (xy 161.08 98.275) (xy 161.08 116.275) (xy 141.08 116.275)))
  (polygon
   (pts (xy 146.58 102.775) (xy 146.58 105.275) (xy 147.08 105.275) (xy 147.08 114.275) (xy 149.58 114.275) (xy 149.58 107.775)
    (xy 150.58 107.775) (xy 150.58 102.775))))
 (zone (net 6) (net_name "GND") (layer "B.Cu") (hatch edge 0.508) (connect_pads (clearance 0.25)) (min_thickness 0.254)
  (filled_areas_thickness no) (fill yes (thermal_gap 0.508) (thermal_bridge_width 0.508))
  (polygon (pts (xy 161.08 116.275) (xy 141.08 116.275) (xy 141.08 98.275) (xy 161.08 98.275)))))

